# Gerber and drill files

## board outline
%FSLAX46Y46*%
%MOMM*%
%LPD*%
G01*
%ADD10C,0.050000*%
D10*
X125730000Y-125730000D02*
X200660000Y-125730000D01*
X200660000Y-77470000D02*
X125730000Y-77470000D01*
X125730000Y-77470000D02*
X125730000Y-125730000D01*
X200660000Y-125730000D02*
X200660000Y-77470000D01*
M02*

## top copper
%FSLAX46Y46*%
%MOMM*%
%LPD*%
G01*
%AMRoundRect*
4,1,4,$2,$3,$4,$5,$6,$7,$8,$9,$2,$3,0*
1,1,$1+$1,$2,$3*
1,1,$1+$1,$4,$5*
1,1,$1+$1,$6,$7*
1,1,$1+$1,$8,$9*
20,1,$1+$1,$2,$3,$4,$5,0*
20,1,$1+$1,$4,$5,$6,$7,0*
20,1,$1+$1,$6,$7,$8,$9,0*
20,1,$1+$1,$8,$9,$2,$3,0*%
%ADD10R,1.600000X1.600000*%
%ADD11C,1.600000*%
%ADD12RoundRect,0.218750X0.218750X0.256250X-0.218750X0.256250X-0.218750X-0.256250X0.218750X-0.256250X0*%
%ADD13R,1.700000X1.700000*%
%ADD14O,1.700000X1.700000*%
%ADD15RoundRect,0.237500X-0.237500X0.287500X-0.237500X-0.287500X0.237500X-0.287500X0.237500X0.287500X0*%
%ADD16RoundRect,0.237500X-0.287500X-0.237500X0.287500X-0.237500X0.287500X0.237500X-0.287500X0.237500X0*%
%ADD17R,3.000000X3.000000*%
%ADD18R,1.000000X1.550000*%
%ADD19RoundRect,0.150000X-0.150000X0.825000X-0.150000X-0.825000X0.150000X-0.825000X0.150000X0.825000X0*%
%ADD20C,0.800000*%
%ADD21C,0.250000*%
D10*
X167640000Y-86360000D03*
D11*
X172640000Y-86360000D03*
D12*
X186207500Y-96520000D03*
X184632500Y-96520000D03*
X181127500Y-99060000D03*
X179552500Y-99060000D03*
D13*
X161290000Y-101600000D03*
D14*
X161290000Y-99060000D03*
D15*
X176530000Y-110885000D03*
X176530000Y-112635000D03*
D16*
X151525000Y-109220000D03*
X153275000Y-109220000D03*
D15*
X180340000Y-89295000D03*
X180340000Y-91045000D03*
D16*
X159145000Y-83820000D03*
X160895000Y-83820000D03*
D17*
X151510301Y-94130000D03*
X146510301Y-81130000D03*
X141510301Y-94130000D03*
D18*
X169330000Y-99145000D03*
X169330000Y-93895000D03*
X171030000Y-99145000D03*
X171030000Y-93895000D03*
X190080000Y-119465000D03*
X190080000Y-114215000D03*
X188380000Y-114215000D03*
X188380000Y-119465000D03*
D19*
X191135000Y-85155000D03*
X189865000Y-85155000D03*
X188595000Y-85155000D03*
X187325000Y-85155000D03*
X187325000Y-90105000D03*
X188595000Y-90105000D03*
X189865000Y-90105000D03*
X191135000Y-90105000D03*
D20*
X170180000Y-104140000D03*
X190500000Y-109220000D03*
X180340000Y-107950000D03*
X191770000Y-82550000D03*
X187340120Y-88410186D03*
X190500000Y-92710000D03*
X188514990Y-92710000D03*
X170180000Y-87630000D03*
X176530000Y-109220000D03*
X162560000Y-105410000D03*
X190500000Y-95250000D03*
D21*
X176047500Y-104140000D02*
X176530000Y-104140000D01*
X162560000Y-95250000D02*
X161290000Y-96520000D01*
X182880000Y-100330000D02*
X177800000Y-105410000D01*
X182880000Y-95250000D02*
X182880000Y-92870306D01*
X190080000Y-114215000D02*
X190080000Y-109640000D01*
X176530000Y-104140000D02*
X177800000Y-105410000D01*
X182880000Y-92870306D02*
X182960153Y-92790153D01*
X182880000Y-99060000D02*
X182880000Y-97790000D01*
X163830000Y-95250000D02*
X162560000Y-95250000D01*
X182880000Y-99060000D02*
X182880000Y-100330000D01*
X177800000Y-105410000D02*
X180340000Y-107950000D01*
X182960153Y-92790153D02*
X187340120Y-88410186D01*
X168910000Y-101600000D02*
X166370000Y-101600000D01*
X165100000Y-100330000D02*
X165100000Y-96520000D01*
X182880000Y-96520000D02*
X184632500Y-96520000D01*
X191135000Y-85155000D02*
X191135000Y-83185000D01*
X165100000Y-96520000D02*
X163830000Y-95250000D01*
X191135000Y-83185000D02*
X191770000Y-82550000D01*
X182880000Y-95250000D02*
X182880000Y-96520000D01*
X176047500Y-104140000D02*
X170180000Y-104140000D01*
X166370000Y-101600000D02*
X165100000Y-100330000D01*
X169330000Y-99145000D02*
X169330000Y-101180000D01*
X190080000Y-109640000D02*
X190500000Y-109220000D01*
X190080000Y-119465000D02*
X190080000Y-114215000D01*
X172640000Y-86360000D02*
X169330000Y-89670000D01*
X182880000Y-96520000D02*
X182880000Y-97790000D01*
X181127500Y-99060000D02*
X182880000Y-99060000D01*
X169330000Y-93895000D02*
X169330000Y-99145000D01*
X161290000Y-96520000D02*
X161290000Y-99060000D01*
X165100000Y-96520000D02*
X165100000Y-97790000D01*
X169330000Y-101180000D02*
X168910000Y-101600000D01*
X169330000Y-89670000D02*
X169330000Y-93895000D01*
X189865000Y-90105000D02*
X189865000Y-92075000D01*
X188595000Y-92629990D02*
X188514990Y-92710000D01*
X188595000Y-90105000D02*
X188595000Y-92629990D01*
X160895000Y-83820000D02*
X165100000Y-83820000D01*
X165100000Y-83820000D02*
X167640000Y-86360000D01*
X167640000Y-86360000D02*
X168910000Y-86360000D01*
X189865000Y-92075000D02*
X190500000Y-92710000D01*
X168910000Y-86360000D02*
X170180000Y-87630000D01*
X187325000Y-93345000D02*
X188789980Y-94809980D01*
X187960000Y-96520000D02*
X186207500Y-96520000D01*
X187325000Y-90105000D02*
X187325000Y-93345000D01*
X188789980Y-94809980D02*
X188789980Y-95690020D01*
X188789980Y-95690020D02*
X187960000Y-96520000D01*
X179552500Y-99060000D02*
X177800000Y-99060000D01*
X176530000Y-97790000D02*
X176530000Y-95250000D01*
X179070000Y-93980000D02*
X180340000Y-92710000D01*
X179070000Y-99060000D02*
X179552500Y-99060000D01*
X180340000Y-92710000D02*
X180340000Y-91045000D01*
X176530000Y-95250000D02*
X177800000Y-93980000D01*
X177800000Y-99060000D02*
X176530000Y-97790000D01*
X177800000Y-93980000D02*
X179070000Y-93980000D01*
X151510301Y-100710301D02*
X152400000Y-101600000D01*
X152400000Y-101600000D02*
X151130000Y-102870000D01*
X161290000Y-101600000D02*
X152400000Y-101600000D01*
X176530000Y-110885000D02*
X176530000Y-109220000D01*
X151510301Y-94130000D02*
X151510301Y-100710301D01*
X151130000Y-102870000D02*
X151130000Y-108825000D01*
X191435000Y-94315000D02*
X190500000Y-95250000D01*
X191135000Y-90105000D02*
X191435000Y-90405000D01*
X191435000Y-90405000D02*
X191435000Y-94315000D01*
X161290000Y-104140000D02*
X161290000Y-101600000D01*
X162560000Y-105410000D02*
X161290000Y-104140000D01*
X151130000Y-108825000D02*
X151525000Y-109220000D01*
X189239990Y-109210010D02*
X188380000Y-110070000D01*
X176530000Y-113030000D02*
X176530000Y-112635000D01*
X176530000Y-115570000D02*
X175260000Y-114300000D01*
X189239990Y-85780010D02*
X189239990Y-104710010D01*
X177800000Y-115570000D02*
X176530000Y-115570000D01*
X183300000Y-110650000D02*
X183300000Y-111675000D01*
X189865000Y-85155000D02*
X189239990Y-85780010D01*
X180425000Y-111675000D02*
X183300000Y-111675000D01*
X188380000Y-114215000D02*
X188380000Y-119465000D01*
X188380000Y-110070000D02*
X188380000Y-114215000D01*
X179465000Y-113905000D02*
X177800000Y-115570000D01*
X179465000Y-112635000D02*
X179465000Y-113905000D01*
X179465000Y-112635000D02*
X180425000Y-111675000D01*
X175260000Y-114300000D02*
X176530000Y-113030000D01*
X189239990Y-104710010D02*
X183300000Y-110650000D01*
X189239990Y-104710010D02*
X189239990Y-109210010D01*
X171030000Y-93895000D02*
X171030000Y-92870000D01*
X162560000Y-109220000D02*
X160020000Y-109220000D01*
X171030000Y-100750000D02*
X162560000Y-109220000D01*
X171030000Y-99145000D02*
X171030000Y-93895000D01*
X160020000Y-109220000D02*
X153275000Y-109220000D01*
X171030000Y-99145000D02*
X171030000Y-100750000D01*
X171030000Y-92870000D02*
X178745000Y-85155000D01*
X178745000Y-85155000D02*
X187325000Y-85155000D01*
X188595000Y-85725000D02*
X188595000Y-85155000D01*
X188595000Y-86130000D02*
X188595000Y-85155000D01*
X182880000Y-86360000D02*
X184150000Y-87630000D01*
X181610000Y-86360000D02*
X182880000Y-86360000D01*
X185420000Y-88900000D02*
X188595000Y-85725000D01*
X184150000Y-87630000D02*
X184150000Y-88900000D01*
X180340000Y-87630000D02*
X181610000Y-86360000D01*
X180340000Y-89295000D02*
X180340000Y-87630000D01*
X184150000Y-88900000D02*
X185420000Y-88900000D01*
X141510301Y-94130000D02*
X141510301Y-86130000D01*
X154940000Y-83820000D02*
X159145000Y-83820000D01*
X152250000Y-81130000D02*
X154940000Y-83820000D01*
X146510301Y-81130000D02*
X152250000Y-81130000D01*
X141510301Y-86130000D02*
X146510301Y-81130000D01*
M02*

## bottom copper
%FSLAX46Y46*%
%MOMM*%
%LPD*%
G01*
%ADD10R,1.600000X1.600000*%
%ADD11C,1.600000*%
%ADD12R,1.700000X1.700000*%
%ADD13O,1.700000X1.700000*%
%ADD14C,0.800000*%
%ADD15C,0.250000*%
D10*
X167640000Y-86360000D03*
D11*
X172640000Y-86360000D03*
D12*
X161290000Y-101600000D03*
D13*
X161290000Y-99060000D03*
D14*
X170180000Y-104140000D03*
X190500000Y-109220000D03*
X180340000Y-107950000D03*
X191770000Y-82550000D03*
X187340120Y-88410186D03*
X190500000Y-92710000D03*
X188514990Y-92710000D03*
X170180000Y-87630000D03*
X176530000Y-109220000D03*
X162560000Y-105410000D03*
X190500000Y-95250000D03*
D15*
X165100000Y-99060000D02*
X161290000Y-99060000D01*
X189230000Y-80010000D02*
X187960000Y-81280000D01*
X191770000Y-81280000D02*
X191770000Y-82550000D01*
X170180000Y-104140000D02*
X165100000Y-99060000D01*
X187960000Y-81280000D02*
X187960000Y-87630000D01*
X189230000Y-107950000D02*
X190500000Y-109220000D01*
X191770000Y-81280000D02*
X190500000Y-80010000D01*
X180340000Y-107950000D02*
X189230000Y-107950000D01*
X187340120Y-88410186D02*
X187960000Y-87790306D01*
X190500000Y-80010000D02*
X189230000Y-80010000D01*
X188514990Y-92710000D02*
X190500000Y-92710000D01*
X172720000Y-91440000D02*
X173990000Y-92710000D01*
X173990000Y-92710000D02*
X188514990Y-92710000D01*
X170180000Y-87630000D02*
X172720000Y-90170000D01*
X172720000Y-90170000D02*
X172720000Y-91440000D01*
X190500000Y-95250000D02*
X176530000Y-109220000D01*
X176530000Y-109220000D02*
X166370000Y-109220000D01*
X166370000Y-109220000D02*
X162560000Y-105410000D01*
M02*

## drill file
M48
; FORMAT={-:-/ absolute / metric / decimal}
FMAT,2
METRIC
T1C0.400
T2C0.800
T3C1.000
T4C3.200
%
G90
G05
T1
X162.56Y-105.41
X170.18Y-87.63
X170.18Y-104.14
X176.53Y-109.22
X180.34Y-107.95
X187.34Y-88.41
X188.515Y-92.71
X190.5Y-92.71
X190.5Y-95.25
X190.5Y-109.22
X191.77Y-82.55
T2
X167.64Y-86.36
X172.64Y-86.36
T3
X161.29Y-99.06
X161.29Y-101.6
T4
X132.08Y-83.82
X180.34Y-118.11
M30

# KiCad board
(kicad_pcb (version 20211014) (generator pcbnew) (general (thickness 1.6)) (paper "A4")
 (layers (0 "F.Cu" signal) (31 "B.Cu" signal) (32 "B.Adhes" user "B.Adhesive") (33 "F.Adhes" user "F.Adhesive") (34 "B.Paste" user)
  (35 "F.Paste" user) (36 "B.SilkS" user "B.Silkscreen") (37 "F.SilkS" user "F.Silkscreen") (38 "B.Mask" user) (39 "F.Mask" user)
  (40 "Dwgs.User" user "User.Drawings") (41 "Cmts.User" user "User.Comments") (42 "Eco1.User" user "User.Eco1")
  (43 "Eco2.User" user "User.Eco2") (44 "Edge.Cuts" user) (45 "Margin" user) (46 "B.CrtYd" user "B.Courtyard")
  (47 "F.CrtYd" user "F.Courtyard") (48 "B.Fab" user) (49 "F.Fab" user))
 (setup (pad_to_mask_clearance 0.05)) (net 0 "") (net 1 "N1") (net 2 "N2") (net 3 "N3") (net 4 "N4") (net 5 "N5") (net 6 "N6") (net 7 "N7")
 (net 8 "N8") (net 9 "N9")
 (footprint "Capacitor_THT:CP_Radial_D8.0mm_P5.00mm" (layer "F.Cu") (at 167.64 86.36)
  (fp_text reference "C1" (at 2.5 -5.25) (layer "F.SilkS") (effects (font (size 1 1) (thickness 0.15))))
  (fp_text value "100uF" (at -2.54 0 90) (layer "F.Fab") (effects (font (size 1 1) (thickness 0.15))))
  (pad "1" thru_hole rect locked (at 0 0) (size 1.6 1.6) (drill 0.8) (layers *.Cu *.Mask) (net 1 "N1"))
  (pad "2" thru_hole circle locked (at 5 0) (size 1.6 1.6) (drill 0.8) (layers *.Cu *.Mask) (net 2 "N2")))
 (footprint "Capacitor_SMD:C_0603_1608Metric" (layer "F.Cu") (at 185.42 96.52 180)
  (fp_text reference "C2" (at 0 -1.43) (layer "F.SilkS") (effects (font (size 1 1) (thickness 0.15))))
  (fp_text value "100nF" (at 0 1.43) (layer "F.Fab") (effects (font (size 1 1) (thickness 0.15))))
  (pad "1" smd roundrect locked (at -0.7875 0 180) (size 0.875 0.95) (layers "F.Cu" "F.Paste" "F.Mask") (roundrect_rratio 0.25) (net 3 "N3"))
  (pad "2" smd roundrect locked (at 0.7875 0 180) (size 0.875 0.95) (layers "F.Cu" "F.Paste" "F.Mask") (roundrect_rratio 0.25) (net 2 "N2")))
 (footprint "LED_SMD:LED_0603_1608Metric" (layer "F.Cu") (at 180.34 99.06 180)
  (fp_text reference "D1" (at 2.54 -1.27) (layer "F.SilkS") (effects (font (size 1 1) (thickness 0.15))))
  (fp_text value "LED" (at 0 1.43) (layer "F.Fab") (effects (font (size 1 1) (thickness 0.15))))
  (pad "1" smd roundrect locked (at -0.7875 0 180) (size 0.875 0.95) (layers "F.Cu" "F.Paste" "F.Mask") (roundrect_rratio 0.25) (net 2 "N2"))
  (pad "2" smd roundrect locked (at 0.7875 0 180) (size 0.875 0.95) (layers "F.Cu" "F.Paste" "F.Mask") (roundrect_rratio 0.25) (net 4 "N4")))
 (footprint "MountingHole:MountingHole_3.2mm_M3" (layer "F.Cu") (at 132.08 83.82)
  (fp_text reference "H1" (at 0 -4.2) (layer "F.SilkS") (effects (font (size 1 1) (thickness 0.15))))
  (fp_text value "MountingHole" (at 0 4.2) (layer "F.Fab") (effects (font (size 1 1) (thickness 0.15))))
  (pad "" np_thru_hole circle locked (at 0 0) (size 3.2 3.2) (drill 3.2) (layers *.Cu *.Mask)))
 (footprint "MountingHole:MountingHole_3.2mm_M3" (layer "F.Cu") (at 180.34 118.11)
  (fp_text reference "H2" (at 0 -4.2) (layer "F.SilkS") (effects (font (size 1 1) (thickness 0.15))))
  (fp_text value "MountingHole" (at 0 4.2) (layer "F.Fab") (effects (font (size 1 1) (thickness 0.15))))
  (pad "" np_thru_hole circle locked (at 0 0) (size 3.2 3.2) (drill 3.2) (layers *.Cu *.Mask)))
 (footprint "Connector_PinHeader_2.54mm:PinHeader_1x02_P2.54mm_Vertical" (layer "F.Cu") (at 161.29 101.6 180)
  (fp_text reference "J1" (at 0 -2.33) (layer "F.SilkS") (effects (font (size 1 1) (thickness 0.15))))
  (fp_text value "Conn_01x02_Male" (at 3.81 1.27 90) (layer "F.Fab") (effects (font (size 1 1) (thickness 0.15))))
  (pad "1" thru_hole rect locked (at 0 0 180) (size 1.7 1.7) (drill 1) (layers *.Cu *.Mask) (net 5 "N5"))
  (pad "2" thru_hole oval locked (at 0 2.54 180) (size 1.7 1.7) (drill 1) (layers *.Cu *.Mask) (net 2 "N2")))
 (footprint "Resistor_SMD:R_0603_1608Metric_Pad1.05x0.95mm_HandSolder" (layer "F.Cu") (at 176.53 111.76 -90)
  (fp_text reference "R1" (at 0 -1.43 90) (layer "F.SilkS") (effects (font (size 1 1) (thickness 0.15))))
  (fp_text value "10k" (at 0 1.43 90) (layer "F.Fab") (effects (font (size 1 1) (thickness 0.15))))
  (pad "1" smd roundrect locked (at -0.875 0 270) (size 1.05 0.95) (layers "F.Cu" "F.Paste" "F.Mask") (roundrect_rratio 0.25) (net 5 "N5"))
  (pad "2" smd roundrect locked (at 0.875 0 270) (size 1.05 0.95) (layers "F.Cu" "F.Paste" "F.Mask") (roundrect_rratio 0.25) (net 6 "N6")))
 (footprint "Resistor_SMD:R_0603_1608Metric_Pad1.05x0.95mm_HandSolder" (layer "F.Cu") (at 152.4 109.22)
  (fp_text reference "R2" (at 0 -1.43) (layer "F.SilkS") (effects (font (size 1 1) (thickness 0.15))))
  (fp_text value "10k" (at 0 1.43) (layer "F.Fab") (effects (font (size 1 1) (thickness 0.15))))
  (pad "1" smd roundrect locked (at -0.875 0) (size 1.05 0.95) (layers "F.Cu" "F.Paste" "F.Mask") (roundrect_rratio 0.25) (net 5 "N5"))
  (pad "2" smd roundrect locked (at 0.875 0) (size 1.05 0.95) (layers "F.Cu" "F.Paste" "F.Mask") (roundrect_rratio 0.25) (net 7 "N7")))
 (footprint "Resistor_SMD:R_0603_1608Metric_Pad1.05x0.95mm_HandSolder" (layer "F.Cu") (at 180.34 90.17 -90)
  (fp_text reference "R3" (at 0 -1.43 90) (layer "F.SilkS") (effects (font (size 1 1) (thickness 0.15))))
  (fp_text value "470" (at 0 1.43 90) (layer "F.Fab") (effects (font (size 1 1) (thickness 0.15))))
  (pad "1" smd roundrect locked (at -0.875 0 270) (size 1.05 0.95) (layers "F.Cu" "F.Paste" "F.Mask") (roundrect_rratio 0.25) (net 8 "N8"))
  (pad "2" smd roundrect locked (at 0.875 0 270) (size 1.05 0.95) (layers "F.Cu" "F.Paste" "F.Mask") (roundrect_rratio 0.25) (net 4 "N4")))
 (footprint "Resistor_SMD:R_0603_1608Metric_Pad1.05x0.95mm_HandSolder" (layer "F.Cu") (at 160.02 83.82)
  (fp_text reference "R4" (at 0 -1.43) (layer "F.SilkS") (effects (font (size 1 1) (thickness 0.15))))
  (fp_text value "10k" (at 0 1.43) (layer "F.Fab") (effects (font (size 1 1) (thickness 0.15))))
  (pad "1" smd roundrect locked (at -0.875 0) (size 1.05 0.95) (layers "F.Cu" "F.Paste" "F.Mask") (roundrect_rratio 0.25) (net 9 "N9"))
  (pad "2" smd roundrect locked (at 0.875 0) (size 1.05 0.95) (layers "F.Cu" "F.Paste" "F.Mask") (roundrect_rratio 0.25) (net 1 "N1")))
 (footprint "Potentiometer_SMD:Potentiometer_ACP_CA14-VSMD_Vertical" (layer "F.Cu") (at 146.510301 87.63 90)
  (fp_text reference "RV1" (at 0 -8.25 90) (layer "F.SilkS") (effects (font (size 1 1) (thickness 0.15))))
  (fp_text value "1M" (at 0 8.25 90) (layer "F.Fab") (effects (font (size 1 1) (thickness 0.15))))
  (pad "1" smd rect locked (at -6.5 5 90) (size 3 3) (layers "F.Cu" "F.Paste" "F.Mask") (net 5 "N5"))
  (pad "2" smd rect locked (at 6.5 0 90) (size 3 3) (layers "F.Cu" "F.Paste" "F.Mask") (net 9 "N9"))
  (pad "3" smd rect locked (at -6.5 -5 90) (size 3 3) (layers "F.Cu" "F.Paste" "F.Mask") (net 9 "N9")))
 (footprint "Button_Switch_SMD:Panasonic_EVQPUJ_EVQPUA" (layer "F.Cu") (at 170.18 96.52 90)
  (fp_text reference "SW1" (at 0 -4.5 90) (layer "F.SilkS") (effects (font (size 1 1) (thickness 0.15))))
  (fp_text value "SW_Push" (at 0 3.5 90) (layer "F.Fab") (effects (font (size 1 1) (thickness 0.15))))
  (pad "1" smd rect locked (at -2.625 -0.85 270) (size 1.55 1) (layers "F.Cu" "F.Paste" "F.Mask") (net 2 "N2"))
  (pad "1" smd rect locked (at 2.625 -0.85 270) (size 1.55 1) (layers "F.Cu" "F.Paste" "F.Mask") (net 2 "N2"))
  (pad "2" smd rect locked (at -2.625 0.85 270) (size 1.55 1) (layers "F.Cu" "F.Paste" "F.Mask") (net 7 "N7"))
  (pad "2" smd rect locked (at 2.625 0.85 270) (size 1.55 1) (layers "F.Cu" "F.Paste" "F.Mask") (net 7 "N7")))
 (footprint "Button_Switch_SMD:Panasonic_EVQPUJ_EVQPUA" (layer "F.Cu") (at 189.23 116.84 -90)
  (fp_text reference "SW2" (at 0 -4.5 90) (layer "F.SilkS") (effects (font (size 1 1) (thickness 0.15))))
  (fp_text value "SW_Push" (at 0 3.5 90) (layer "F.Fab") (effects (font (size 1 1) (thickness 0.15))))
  (pad "1" smd rect locked (at 2.625 -0.85 90) (size 1.55 1) (layers "F.Cu" "F.Paste" "F.Mask") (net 2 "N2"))
  (pad "1" smd rect locked (at -2.625 -0.85 90) (size 1.55 1) (layers "F.Cu" "F.Paste" "F.Mask") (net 2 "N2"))
  (pad "2" smd rect locked (at -2.625 0.85 90) (size 1.55 1) (layers "F.Cu" "F.Paste" "F.Mask") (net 6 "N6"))
  (pad "2" smd rect locked (at 2.625 0.85 90) (size 1.55 1) (layers "F.Cu" "F.Paste" "F.Mask") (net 6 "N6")))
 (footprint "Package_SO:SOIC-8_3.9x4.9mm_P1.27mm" (layer "F.Cu") (at 189.23 87.63 -90)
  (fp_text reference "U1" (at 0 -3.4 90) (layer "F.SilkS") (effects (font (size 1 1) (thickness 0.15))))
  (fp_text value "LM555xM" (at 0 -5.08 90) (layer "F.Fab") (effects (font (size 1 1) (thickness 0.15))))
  (pad "1" smd roundrect locked (at -2.475 -1.905 270) (size 1.95 0.6) (layers "F.Cu" "F.Paste" "F.Mask") (roundrect_rratio 0.25)
   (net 2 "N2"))
  (pad "2" smd roundrect locked (at -2.475 -0.635 270) (size 1.95 0.6) (layers "F.Cu" "F.Paste" "F.Mask") (roundrect_rratio 0.25)
   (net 6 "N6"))
  (pad "3" smd roundrect locked (at -2.475 0.635 270) (size 1.95 0.6) (layers "F.Cu" "F.Paste" "F.Mask") (roundrect_rratio 0.25)
   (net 8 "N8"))
  (pad "4" smd roundrect locked (at -2.475 1.905 270) (size 1.95 0.6) (layers "F.Cu" "F.Paste" "F.Mask") (roundrect_rratio 0.25)
   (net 7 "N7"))
  (pad "5" smd roundrect locked (at 2.475 1.905 270) (size 1.95 0.6) (layers "F.Cu" "F.Paste" "F.Mask") (roundrect_rratio 0.25) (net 3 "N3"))
  (pad "6" smd roundrect locked (at 2.475 0.635 270) (size 1.95 0.6) (layers "F.Cu" "F.Paste" "F.Mask") (roundrect_rratio 0.25) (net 1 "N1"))
  (pad "7" smd roundrect locked (at 2.475 -0.635 270) (size 1.95 0.6) (layers "F.Cu" "F.Paste" "F.Mask") (roundrect_rratio 0.25)
   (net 1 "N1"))
  (pad "8" smd roundrect locked (at 2.475 -1.905 270) (size 1.95 0.6) (layers "F.Cu" "F.Paste" "F.Mask") (roundrect_rratio 0.25)
   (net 5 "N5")))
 (gr_line (start 125.73 125.73) (end 200.66 125.73) (layer "Edge.Cuts") (width 0.05))
 (gr_line (start 200.66 77.47) (end 125.73 77.47) (layer "Edge.Cuts") (width 0.05))
 (gr_line (start 125.73 77.47) (end 125.73 125.73) (layer "Edge.Cuts") (width 0.05))
 (gr_line (start 200.66 125.73) (end 200.66 77.47) (layer "Edge.Cuts") (width 0.05))
 (segment (start 176.0475 104.14) (end 176.53 104.14) (width 0.25) (layer "F.Cu") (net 2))
 (segment (start 162.56 95.25) (end 161.29 96.52) (width 0.25) (layer "F.Cu") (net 2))
 (segment (start 182.88 100.33) (end 177.8 105.41) (width 0.25) (layer "F.Cu") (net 2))
 (segment (start 182.88 95.25) (end 182.88 92.870306) (width 0.25) (layer "F.Cu") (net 2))
 (segment (start 190.08 114.215) (end 190.08 109.64) (width 0.25) (layer "F.Cu") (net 2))
 (segment (start 176.53 104.14) (end 177.8 105.41) (width 0.25) (layer "F.Cu") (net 2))
 (segment (start 182.88 92.870306) (end 182.960153 92.790153) (width 0.25) (layer "F.Cu") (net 2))
 (segment (start 182.88 99.06) (end 182.88 97.79) (width 0.25) (layer "F.Cu") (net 2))
 (segment (start 163.83 95.25) (end 162.56 95.25) (width 0.25) (layer "F.Cu") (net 2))
 (segment (start 182.88 99.06) (end 182.88 100.33) (width 0.25) (layer "F.Cu") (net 2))
 (segment (start 177.8 105.41) (end 180.34 107.95) (width 0.25) (layer "F.Cu") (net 2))
 (segment (start 182.960153 92.790153) (end 187.34012 88.410186) (width 0.25) (layer "F.Cu") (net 2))
 (segment (start 168.91 101.6) (end 166.37 101.6) (width 0.25) (layer "F.Cu") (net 2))
 (segment (start 165.1 100.33) (end 165.1 96.52) (width 0.25) (layer "F.Cu") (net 2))
 (segment (start 182.88 96.52) (end 184.6325 96.52) (width 0.25) (layer "F.Cu") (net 2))
 (segment (start 191.135 85.155) (end 191.135 83.185) (width 0.25) (layer "F.Cu") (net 2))
 (segment (start 165.1 96.52) (end 163.83 95.25) (width 0.25) (layer "F.Cu") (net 2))
 (segment (start 191.135 83.185) (end 191.77 82.55) (width 0.25) (layer "F.Cu") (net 2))
 (segment (start 182.88 95.25) (end 182.88 96.52) (width 0.25) (layer "F.Cu") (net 2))
 (segment (start 176.0475 104.14) (end 170.18 104.14) (width 0.25) (layer "F.Cu") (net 2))
 (segment (start 166.37 101.6) (end 165.1 100.33) (width 0.25) (layer "F.Cu") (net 2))
 (segment (start 169.33 99.145) (end 169.33 101.18) (width 0.25) (layer "F.Cu") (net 2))
 (segment (start 190.08 109.64) (end 190.5 109.22) (width 0.25) (layer "F.Cu") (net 2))
 (segment (start 190.08 119.465) (end 190.08 114.215) (width 0.25) (layer "F.Cu") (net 2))
 (segment (start 172.64 86.36) (end 169.33 89.67) (width 0.25) (layer "F.Cu") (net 2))
 (segment (start 182.88 96.52) (end 182.88 97.79) (width 0.25) (layer "F.Cu") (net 2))
 (segment (start 181.1275 99.06) (end 182.88 99.06) (width 0.25) (layer "F.Cu") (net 2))
 (segment (start 169.33 93.895) (end 169.33 99.145) (width 0.25) (layer "F.Cu") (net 2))
 (segment (start 161.29 96.52) (end 161.29 99.06) (width 0.25) (layer "F.Cu") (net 2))
 (segment (start 165.1 96.52) (end 165.1 97.79) (width 0.25) (layer "F.Cu") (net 2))
 (segment (start 169.33 101.18) (end 168.91 101.6) (width 0.25) (layer "F.Cu") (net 2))
 (segment (start 169.33 89.67) (end 169.33 93.895) (width 0.25) (layer "F.Cu") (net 2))
 (via (at 170.18 104.14) (size 0.8) (drill 0.4) (layers "F.Cu" "B.Cu") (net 2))
 (via (at 190.5 109.22) (size 0.8) (drill 0.4) (layers "F.Cu" "B.Cu") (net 2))
 (via (at 180.34 107.95) (size 0.8) (drill 0.4) (layers "F.Cu" "B.Cu") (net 2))
 (via (at 191.77 82.55) (size 0.8) (drill 0.4) (layers "F.Cu" "B.Cu") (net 2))
 (via (at 187.34012 88.410186) (size 0.8) (drill 0.4) (layers "F.Cu" "B.Cu") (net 2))
 (segment (start 165.1 99.06) (end 161.29 99.06) (width 0.25) (layer "B.Cu") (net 2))
 (segment (start 189.23 80.01) (end 187.96 81.28) (width 0.25) (layer "B.Cu") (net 2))
 (segment (start 191.77 81.28) (end 191.77 82.55) (width 0.25) (layer "B.Cu") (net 2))
 (segment (start 170.18 104.14) (end 165.1 99.06) (width 0.25) (layer "B.Cu") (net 2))
 (segment (start 187.96 81.28) (end 187.96 87.63) (width 0.25) (layer "B.Cu") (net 2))
 (segment (start 189.23 107.95) (end 190.5 109.22) (width 0.25) (layer "B.Cu") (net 2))
 (segment (start 191.77 81.28) (end 190.5 80.01) (width 0.25) (layer "B.Cu") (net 2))
 (segment (start 180.34 107.95) (end 189.23 107.95) (width 0.25) (layer "B.Cu") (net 2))
 (segment (start 187.34012 88.410186) (end 187.96 87.790306) (width 0.25) (layer "B.Cu") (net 2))
 (segment (start 190.5 80.01) (end 189.23 80.01) (width 0.25) (layer "B.Cu") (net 2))
 (segment (start 189.865 90.105) (end 189.865 92.075) (width 0.25) (layer "F.Cu") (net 1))
 (segment (start 188.595 92.62999) (end 188.51499 92.71) (width 0.25) (layer "F.Cu") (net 1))
 (segment (start 188.595 90.105) (end 188.595 92.62999) (width 0.25) (layer "F.Cu") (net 1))
 (segment (start 160.895 83.82) (end 165.1 83.82) (width 0.25) (layer "F.Cu") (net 1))
 (segment (start 165.1 83.82) (end 167.64 86.36) (width 0.25) (layer "F.Cu") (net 1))
 (segment (start 167.64 86.36) (end 168.91 86.36) (width 0.25) (layer "F.Cu") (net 1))
 (segment (start 189.865 92.075) (end 190.5 92.71) (width 0.25) (layer "F.Cu") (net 1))
 (segment (start 168.91 86.36) (end 170.18 87.63) (width 0.25) (layer "F.Cu") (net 1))
 (via (at 190.5 92.71) (size 0.8) (drill 0.4) (layers "F.Cu" "B.Cu") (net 1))
 (via (at 188.51499 92.71) (size 0.8) (drill 0.4) (layers "F.Cu" "B.Cu") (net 1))
 (via (at 170.18 87.63) (size 0.8) (drill 0.4) (layers "F.Cu" "B.Cu") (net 1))
 (segment (start 188.51499 92.71) (end 190.5 92.71) (width 0.25) (layer "B.Cu") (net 1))
 (segment (start 172.72 91.44) (end 173.99 92.71) (width 0.25) (layer "B.Cu") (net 1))
 (segment (start 173.99 92.71) (end 188.51499 92.71) (width 0.25) (layer "B.Cu") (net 1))
 (segment (start 170.18 87.63) (end 172.72 90.17) (width 0.25) (layer "B.Cu") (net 1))
 (segment (start 172.72 90.17) (end 172.72 91.44) (width 0.25) (layer "B.Cu") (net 1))
 (segment (start 187.325 93.345) (end 188.78998 94.80998) (width 0.25) (layer "F.Cu") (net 3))
 (segment (start 187.96 96.52) (end 186.2075 96.52) (width 0.25) (layer "F.Cu") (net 3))
 (segment (start 187.325 90.105) (end 187.325 93.345) (width 0.25) (layer "F.Cu") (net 3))
 (segment (start 188.78998 94.80998) (end 188.78998 95.69002) (width 0.25) (layer "F.Cu") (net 3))
 (segment (start 188.78998 95.69002) (end 187.96 96.52) (width 0.25) (layer "F.Cu") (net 3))
 (segment (start 179.5525 99.06) (end 177.8 99.06) (width 0.25) (layer "F.Cu") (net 4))
 (segment (start 176.53 97.79) (end 176.53 95.25) (width 0.25) (layer "F.Cu") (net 4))
 (segment (start 179.07 93.98) (end 180.34 92.71) (width 0.25) (layer "F.Cu") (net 4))
 (segment (start 179.07 99.06) (end 179.5525 99.06) (width 0.25) (layer "F.Cu") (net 4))
 (segment (start 180.34 92.71) (end 180.34 91.045) (width 0.25) (layer "F.Cu") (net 4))
 (segment (start 176.53 95.25) (end 177.8 93.98) (width 0.25) (layer "F.Cu") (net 4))
 (segment (start 177.8 99.06) (end 176.53 97.79) (width 0.25) (layer "F.Cu") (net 4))
 (segment (start 177.8 93.98) (end 179.07 93.98) (width 0.25) (layer "F.Cu") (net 4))
 (segment (start 151.510301 100.710301) (end 152.4 101.6) (width 0.25) (layer "F.Cu") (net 5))
 (segment (start 152.4 101.6) (end 151.13 102.87) (width 0.25) (layer "F.Cu") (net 5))
 (segment (start 161.29 101.6) (end 152.4 101.6) (width 0.25) (layer "F.Cu") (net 5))
 (segment (start 176.53 110.885) (end 176.53 109.22) (width 0.25) (layer "F.Cu") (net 5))
 (segment (start 151.510301 94.13) (end 151.510301 100.710301) (width 0.25) (layer "F.Cu") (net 5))
 (segment (start 151.13 102.87) (end 151.13 108.825) (width 0.25) (layer "F.Cu") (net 5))
 (segment (start 191.435 94.315) (end 190.5 95.25) (width 0.25) (layer "F.Cu") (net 5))
 (segment (start 191.135 90.105) (end 191.435 90.405) (width 0.25) (layer "F.Cu") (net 5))
 (segment (start 191.435 90.405) (end 191.435 94.315) (width 0.25) (layer "F.Cu") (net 5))
 (segment (start 161.29 104.14) (end 161.29 101.6) (width 0.25) (layer "F.Cu") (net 5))
 (segment (start 162.56 105.41) (end 161.29 104.14) (width 0.25) (layer "F.Cu") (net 5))
 (segment (start 151.13 108.825) (end 151.525 109.22) (width 0.25) (layer "F.Cu") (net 5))
 (via (at 176.53 109.22) (size 0.8) (drill 0.4) (layers "F.Cu" "B.Cu") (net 5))
 (via (at 162.56 105.41) (size 0.8) (drill 0.4) (layers "F.Cu" "B.Cu") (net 5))
 (via (at 190.5 95.25) (size 0.8) (drill 0.4) (layers "F.Cu" "B.Cu") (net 5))
 (segment (start 190.5 95.25) (end 176.53 109.22) (width 0.25) (layer "B.Cu") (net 5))
 (segment (start 176.53 109.22) (end 166.37 109.22) (width 0.25) (layer "B.Cu") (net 5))
 (segment (start 166.37 109.22) (end 162.56 105.41) (width 0.25) (layer "B.Cu") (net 5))
 (segment (start 189.23999 109.21001) (end 188.38 110.07) (width 0.25) (layer "F.Cu") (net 6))
 (segment (start 176.53 113.03) (end 176.53 112.635) (width 0.25) (layer "F.Cu") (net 6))
 (segment (start 176.53 115.57) (end 175.26 114.3) (width 0.25) (layer "F.Cu") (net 6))
 (segment (start 189.23999 85.78001) (end 189.23999 104.71001) (width 0.25) (layer "F.Cu") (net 6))
 (segment (start 177.8 115.57) (end 176.53 115.57) (width 0.25) (layer "F.Cu") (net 6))
 (segment (start 183.3 110.65) (end 183.3 111.675) (width 0.25) (layer "F.Cu") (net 6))
 (segment (start 189.865 85.155) (end 189.23999 85.78001) (width 0.25) (layer "F.Cu") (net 6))
 (segment (start 180.425 111.675) (end 183.3 111.675) (width 0.25) (layer "F.Cu") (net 6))
 (segment (start 188.38 114.215) (end 188.38 119.465) (width 0.25) (layer "F.Cu") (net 6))
 (segment (start 188.38 110.07) (end 188.38 114.215) (width 0.25) (layer "F.Cu") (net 6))
 (segment (start 179.465 113.905) (end 177.8 115.57) (width 0.25) (layer "F.Cu") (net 6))
 (segment (start 179.465 112.635) (end 179.465 113.905) (width 0.25) (layer "F.Cu") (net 6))
 (segment (start 179.465 112.635) (end 180.425 111.675) (width 0.25) (layer "F.Cu") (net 6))
 (segment (start 175.26 114.3) (end 176.53 113.03) (width 0.25) (layer "F.Cu") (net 6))
 (segment (start 189.23999 104.71001) (end 183.3 110.65) (width 0.25) (layer "F.Cu") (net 6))
 (segment (start 189.23999 104.71001) (end 189.23999 109.21001) (width 0.25) (layer "F.Cu") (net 6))
 (segment (start 171.03 93.895) (end 171.03 92.87) (width 0.25) (layer "F.Cu") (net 7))
 (segment (start 162.56 109.22) (end 160.02 109.22) (width 0.25) (layer "F.Cu") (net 7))
 (segment (start 171.03 100.75) (end 162.56 109.22) (width 0.25) (layer "F.Cu") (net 7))
 (segment (start 171.03 99.145) (end 171.03 93.895) (width 0.25) (layer "F.Cu") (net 7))
 (segment (start 160.02 109.22) (end 153.275 109.22) (width 0.25) (layer "F.Cu") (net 7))
 (segment (start 171.03 99.145) (end 171.03 100.75) (width 0.25) (layer "F.Cu") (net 7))
 (segment (start 171.03 92.87) (end 178.745 85.155) (width 0.25) (layer "F.Cu") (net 7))
 (segment (start 178.745 85.155) (end 187.325 85.155) (width 0.25) (layer "F.Cu") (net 7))
 (segment (start 188.595 85.725) (end 188.595 85.155) (width 0.25) (layer "F.Cu") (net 8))
 (segment (start 188.595 86.13) (end 188.595 85.155) (width 0.25) (layer "F.Cu") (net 8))
 (segment (start 182.88 86.36) (end 184.15 87.63) (width 0.25) (layer "F.Cu") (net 8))
 (segment (start 181.61 86.36) (end 182.88 86.36) (width 0.25) (layer "F.Cu") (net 8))
 (segment (start 185.42 88.9) (end 188.595 85.725) (width 0.25) (layer "F.Cu") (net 8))
 (segment (start 184.15 87.63) (end 184.15 88.9) (width 0.25) (layer "F.Cu") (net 8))
 (segment (start 180.34 87.63) (end 181.61 86.36) (width 0.25) (layer "F.Cu") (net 8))
 (segment (start 180.34 89.295) (end 180.34 87.63) (width 0.25) (layer "F.Cu") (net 8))
 (segment (start 184.15 88.9) (end 185.42 88.9) (width 0.25) (layer "F.Cu") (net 8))
 (segment (start 141.510301 94.13) (end 141.510301 86.13) (width 0.25) (layer "F.Cu") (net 9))
 (segment (start 154.94 83.82) (end 159.145 83.82) (width 0.25) (layer "F.Cu") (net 9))
 (segment (start 152.25 81.13) (end 154.94 83.82) (width 0.25) (layer "F.Cu") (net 9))
 (segment (start 146.510301 81.13) (end 152.25 81.13) (width 0.25) (layer "F.Cu") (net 9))
 (segment (start 141.510301 86.13) (end 146.510301 81.13) (width 0.25) (layer "F.Cu") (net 9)))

